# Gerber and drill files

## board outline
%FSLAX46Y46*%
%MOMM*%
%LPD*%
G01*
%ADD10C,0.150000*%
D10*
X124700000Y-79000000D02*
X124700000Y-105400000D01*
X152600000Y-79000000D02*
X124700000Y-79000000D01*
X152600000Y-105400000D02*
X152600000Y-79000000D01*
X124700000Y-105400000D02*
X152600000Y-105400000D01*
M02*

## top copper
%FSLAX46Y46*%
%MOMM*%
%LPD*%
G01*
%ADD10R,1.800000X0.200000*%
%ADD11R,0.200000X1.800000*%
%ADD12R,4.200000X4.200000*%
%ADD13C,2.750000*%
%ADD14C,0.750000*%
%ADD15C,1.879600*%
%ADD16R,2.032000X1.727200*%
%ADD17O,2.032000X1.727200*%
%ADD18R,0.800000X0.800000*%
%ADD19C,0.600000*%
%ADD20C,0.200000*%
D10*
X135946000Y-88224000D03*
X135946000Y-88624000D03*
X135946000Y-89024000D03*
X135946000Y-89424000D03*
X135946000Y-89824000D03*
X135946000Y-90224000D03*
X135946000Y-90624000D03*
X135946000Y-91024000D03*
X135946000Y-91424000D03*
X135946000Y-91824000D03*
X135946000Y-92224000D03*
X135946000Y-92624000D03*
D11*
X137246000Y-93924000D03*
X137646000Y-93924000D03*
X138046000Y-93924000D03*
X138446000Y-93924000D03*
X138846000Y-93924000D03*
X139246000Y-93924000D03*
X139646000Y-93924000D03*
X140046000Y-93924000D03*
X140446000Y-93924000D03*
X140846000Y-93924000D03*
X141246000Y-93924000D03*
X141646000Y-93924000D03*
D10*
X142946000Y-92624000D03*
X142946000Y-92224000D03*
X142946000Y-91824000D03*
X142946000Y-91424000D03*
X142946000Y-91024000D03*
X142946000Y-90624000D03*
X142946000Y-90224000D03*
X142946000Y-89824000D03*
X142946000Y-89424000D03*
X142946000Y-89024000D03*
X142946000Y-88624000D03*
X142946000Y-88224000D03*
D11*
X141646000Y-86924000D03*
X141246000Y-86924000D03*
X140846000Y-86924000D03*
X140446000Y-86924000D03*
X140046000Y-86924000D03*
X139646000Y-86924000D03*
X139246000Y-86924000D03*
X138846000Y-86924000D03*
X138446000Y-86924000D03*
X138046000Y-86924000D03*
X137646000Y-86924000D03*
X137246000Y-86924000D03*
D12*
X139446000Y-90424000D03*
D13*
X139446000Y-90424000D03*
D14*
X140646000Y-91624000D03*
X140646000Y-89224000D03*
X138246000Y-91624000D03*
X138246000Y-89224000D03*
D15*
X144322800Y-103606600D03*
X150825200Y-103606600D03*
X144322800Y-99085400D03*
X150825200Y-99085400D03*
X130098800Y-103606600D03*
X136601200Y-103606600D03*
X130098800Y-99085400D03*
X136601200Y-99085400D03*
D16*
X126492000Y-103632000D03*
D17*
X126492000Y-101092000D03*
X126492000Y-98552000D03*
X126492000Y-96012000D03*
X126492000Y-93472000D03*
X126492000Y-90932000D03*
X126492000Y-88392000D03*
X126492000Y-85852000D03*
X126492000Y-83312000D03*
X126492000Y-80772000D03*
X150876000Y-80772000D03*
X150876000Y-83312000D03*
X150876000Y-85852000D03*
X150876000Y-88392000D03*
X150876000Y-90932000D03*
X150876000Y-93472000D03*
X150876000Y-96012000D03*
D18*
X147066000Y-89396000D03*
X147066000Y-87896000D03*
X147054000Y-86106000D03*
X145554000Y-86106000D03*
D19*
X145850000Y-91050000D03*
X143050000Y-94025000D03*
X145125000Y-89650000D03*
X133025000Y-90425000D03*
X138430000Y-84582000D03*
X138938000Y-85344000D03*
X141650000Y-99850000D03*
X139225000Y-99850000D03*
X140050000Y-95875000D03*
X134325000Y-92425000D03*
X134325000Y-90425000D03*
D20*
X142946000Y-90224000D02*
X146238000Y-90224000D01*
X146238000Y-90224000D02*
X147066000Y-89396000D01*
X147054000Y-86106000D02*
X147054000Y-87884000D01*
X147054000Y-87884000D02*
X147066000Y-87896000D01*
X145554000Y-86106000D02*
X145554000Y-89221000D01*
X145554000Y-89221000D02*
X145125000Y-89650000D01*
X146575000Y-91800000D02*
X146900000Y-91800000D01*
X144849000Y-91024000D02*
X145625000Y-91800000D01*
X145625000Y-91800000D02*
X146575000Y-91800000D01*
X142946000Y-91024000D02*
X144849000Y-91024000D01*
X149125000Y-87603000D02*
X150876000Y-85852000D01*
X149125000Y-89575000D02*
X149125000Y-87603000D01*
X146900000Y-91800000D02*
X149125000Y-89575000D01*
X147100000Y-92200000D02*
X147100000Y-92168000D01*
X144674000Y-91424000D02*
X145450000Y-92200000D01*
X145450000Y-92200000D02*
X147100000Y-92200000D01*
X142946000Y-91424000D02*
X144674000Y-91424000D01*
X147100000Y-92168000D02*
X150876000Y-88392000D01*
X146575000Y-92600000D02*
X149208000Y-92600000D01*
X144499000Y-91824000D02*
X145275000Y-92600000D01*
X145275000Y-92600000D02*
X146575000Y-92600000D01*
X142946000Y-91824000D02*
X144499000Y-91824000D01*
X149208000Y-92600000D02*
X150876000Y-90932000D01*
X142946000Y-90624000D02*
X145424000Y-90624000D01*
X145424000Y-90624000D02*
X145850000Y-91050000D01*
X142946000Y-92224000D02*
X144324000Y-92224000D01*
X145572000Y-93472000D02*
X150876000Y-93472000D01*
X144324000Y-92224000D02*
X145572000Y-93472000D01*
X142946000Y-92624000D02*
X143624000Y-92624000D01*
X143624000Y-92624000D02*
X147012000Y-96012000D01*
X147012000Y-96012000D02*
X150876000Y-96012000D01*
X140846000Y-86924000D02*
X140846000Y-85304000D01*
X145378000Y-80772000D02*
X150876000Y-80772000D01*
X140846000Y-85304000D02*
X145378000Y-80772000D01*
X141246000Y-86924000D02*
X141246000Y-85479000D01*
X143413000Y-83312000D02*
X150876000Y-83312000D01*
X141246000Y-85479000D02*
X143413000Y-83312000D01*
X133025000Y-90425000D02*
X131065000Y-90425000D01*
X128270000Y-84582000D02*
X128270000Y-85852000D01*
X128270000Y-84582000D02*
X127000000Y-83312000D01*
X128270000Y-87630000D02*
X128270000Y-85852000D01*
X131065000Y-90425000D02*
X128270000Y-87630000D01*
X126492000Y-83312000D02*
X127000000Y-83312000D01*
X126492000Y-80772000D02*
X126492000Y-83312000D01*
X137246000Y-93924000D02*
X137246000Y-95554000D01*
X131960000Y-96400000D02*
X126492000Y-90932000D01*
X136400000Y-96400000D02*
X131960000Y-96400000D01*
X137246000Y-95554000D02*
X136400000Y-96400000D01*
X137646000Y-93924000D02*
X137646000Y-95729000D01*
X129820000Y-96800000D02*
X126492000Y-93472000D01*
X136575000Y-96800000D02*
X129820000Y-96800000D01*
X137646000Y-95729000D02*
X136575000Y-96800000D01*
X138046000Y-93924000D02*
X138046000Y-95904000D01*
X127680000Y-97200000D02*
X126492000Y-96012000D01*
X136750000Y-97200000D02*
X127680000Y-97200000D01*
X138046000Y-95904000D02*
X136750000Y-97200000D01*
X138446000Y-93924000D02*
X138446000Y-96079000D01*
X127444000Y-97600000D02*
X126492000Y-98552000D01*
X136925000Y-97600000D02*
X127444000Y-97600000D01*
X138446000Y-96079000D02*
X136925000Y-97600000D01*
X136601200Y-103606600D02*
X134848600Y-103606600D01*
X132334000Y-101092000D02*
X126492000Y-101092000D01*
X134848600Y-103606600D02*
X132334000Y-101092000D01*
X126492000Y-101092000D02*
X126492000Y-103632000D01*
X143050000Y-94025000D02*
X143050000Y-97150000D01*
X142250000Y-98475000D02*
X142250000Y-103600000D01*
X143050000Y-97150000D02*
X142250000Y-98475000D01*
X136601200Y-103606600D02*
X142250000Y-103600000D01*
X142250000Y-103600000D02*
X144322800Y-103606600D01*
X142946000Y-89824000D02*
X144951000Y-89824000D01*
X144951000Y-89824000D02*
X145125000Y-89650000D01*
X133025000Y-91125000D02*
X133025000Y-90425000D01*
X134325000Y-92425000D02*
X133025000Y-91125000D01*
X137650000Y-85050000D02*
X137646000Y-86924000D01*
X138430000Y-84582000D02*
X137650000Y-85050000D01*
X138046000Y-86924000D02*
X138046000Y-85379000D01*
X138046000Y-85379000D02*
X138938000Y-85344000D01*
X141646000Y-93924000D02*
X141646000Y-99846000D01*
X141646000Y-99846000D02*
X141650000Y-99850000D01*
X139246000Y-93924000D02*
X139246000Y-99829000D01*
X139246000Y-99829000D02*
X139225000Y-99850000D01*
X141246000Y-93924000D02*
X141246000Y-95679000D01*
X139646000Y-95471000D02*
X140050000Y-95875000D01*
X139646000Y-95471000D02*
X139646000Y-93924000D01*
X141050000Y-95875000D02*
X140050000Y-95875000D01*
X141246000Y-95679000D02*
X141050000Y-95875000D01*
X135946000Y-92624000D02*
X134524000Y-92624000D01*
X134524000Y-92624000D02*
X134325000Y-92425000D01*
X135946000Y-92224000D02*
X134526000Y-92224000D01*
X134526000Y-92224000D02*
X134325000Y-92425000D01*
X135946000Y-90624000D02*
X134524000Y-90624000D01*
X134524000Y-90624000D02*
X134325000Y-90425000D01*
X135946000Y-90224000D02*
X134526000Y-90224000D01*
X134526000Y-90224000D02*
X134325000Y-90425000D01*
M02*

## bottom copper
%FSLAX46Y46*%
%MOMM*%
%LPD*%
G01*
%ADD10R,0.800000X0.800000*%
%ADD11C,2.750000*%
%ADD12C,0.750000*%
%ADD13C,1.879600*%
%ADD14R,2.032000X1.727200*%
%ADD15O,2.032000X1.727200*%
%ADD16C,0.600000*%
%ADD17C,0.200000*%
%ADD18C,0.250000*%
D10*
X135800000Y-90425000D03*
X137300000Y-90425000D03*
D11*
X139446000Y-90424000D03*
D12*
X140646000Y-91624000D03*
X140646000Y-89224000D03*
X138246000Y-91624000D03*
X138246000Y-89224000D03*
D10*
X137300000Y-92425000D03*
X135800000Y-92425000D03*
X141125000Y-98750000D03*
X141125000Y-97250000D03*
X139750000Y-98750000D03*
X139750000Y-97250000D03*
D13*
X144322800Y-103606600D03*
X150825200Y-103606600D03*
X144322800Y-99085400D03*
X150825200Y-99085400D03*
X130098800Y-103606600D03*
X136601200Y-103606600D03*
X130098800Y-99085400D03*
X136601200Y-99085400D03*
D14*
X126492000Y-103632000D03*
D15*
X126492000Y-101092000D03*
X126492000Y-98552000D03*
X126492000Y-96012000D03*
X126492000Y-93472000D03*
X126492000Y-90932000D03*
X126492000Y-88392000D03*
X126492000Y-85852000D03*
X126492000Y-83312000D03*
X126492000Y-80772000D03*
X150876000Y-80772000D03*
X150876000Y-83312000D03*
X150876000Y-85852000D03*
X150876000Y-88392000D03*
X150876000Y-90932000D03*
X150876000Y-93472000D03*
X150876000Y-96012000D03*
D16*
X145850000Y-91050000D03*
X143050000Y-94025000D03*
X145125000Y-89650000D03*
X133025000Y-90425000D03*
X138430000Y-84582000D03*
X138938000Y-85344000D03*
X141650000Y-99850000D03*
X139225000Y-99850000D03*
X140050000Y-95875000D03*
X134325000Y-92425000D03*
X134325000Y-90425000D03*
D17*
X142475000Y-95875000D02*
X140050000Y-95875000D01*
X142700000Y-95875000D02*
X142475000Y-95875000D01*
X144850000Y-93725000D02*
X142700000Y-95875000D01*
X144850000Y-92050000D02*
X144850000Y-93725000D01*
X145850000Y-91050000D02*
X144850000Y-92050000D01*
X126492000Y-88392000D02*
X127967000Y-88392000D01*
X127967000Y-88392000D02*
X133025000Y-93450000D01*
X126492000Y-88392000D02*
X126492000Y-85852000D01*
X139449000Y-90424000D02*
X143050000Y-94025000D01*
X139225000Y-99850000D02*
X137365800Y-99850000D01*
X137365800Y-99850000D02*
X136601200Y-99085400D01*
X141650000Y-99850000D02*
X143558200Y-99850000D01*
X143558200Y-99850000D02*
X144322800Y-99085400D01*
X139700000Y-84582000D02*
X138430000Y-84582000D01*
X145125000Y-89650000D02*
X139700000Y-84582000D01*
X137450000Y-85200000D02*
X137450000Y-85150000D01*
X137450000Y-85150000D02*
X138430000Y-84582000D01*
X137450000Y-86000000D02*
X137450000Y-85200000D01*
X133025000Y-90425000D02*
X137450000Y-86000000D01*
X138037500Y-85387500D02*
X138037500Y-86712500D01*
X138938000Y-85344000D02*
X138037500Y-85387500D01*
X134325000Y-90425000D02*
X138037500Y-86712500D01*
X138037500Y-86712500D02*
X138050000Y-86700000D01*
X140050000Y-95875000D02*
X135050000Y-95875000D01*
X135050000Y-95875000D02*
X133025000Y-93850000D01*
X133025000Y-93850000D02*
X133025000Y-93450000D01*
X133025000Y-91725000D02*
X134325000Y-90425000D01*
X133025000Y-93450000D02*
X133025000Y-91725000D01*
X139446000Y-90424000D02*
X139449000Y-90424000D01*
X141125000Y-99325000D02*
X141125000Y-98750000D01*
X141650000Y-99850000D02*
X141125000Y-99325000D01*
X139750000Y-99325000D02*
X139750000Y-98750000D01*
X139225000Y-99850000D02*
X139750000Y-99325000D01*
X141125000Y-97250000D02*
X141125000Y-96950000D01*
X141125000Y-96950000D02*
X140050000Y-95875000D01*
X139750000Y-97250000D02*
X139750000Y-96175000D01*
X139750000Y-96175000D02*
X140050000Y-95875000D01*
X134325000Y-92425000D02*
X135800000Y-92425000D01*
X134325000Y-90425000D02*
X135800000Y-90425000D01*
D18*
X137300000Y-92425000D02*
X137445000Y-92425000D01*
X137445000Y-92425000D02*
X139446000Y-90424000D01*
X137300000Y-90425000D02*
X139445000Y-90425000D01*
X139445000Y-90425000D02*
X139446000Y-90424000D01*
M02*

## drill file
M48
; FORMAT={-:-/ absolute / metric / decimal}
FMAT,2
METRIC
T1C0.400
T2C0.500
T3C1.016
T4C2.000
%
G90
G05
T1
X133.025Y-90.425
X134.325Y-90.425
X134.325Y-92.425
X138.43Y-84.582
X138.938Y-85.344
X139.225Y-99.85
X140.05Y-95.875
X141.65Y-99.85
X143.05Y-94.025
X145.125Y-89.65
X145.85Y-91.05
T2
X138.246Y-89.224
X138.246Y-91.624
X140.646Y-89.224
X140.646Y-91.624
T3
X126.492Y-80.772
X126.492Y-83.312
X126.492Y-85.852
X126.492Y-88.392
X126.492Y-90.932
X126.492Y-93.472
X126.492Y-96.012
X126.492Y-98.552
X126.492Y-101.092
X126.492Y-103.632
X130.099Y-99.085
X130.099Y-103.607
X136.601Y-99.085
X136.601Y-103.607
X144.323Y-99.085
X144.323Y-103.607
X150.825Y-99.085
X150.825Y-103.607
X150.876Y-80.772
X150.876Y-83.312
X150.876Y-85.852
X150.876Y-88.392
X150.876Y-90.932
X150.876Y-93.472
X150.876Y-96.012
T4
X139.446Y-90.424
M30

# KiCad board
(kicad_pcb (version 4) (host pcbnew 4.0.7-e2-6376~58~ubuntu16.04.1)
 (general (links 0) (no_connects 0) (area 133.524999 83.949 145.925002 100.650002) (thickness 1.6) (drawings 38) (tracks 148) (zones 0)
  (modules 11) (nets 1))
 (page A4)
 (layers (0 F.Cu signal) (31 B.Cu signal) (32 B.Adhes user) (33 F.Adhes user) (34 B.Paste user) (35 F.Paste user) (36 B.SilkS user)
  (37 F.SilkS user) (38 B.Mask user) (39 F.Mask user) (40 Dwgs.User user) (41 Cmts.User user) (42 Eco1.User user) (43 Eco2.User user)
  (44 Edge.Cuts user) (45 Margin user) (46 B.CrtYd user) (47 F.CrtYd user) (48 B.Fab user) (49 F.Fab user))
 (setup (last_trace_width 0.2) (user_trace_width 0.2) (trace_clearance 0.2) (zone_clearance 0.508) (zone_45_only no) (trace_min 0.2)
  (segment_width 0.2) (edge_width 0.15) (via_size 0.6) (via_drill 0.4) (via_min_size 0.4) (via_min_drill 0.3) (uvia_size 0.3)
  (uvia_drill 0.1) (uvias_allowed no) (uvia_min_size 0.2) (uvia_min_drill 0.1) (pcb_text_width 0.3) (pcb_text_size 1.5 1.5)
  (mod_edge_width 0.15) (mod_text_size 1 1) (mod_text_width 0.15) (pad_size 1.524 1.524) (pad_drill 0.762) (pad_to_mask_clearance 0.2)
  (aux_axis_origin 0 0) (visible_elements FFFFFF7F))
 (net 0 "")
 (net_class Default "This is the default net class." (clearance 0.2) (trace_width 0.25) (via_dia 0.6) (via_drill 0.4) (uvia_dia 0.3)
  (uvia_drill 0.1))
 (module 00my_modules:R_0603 (layer B.Cu) (at 136.55 90.425)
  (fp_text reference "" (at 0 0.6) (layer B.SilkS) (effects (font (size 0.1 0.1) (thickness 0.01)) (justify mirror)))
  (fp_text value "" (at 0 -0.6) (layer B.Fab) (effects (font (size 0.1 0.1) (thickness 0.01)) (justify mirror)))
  (pad 1 smd rect (at -0.75 0) (size 0.8 0.8) (layers B.Cu B.Paste B.Mask))
  (pad 2 smd rect (at 0.75 0) (size 0.8 0.8) (layers B.Cu B.Paste B.Mask)))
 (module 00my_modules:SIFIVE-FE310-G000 (layer F.Cu) (at 139.446 90.424)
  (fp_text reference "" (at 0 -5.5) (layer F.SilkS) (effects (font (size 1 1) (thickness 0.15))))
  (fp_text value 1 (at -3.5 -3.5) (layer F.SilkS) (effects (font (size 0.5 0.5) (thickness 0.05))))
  (pad DQ3 smd rect (at -3.5 -2.2) (size 1.8 0.2) (layers F.Cu F.Paste F.Mask))
  (pad DQ2 smd rect (at -3.5 -1.8) (size 1.8 0.2) (layers F.Cu F.Paste F.Mask))
  (pad DQ1 smd rect (at -3.5 -1.4) (size 1.8 0.2) (layers F.Cu F.Paste F.Mask))
  (pad DQ0 smd rect (at -3.5 -1) (size 1.8 0.2) (layers F.Cu F.Paste F.Mask))
  (pad CS smd rect (at -3.5 -0.6) (size 1.8 0.2) (layers F.Cu F.Paste F.Mask))
  (pad 1.8V smd rect (at -3.5 -0.2) (size 1.8 0.2) (layers F.Cu F.Paste F.Mask))
  (pad 1.8V smd rect (at -3.5 0.2) (size 1.8 0.2) (layers F.Cu F.Paste F.Mask))
  (pad PLL smd rect (at -3.5 0.6) (size 1.8 0.2) (layers F.Cu F.Paste F.Mask))
  (pad XIN smd rect (at -3.5 1) (size 1.8 0.2) (layers F.Cu F.Paste F.Mask))
  (pad NC smd rect (at -3.5 1.4) (size 1.8 0.2) (layers F.Cu F.Paste F.Mask))
  (pad 3.3V smd rect (at -3.5 1.8) (size 1.8 0.2) (layers F.Cu F.Paste F.Mask))
  (pad 3.3V smd rect (at -3.5 2.2) (size 1.8 0.2) (layers F.Cu F.Paste F.Mask))
  (pad TCK smd rect (at -2.2 3.5 90) (size 1.8 0.2) (layers F.Cu F.Paste F.Mask))
  (pad TDO smd rect (at -1.8 3.5 90) (size 1.8 0.2) (layers F.Cu F.Paste F.Mask))
  (pad TMS smd rect (at -1.4 3.5 90) (size 1.8 0.2) (layers F.Cu F.Paste F.Mask))
  (pad TDI smd rect (at -1 3.5 90) (size 1.8 0.2) (layers F.Cu F.Paste F.Mask))
  (pad 17 smd rect (at -0.6 3.5 90) (size 1.8 0.2) (layers F.Cu F.Paste F.Mask))
  (pad WAKE smd rect (at -0.2 3.5 90) (size 1.8 0.2) (layers F.Cu F.Paste F.Mask))
  (pad 1.8V smd rect (at 0.2 3.5 90) (size 1.8 0.2) (layers F.Cu F.Paste F.Mask))
  (pad 20 smd rect (at 0.6 3.5 90) (size 1.8 0.2) (layers F.Cu F.Paste F.Mask))
  (pad 21 smd rect (at 1 3.5 90) (size 1.8 0.2) (layers F.Cu F.Paste F.Mask))
  (pad 22 smd rect (at 1.4 3.5 90) (size 1.8 0.2) (layers F.Cu F.Paste F.Mask))
  (pad 1.8V smd rect (at 1.8 3.5 90) (size 1.8 0.2) (layers F.Cu F.Paste F.Mask))
  (pad ERST smd rect (at 2.2 3.5 90) (size 1.8 0.2) (layers F.Cu F.Paste F.Mask))
  (pad G00 smd rect (at 3.5 2.2) (size 1.8 0.2) (layers F.Cu F.Paste F.Mask))
  (pad G01 smd rect (at 3.5 1.8) (size 1.8 0.2) (layers F.Cu F.Paste F.Mask))
  (pad G02 smd rect (at 3.5 1.4) (size 1.8 0.2) (layers F.Cu F.Paste F.Mask))
  (pad G03 smd rect (at 3.5 1) (size 1.8 0.2) (layers F.Cu F.Paste F.Mask))
  (pad G04 smd rect (at 3.5 0.6) (size 1.8 0.2) (layers F.Cu F.Paste F.Mask))
  (pad 1.8V smd rect (at 3.5 0.2) (size 1.8 0.2) (layers F.Cu F.Paste F.Mask))
  (pad G05 smd rect (at 3.5 -0.2) (size 1.8 0.2) (layers F.Cu F.Paste F.Mask))
  (pad 3.3V smd rect (at 3.5 -0.6) (size 1.8 0.2) (layers F.Cu F.Paste F.Mask))
  (pad G09 smd rect (at 3.5 -1) (size 1.8 0.2) (layers F.Cu F.Paste F.Mask))
  (pad G10 smd rect (at 3.5 -1.4) (size 1.8 0.2) (layers F.Cu F.Paste F.Mask))
  (pad G11 smd rect (at 3.5 -1.8) (size 1.8 0.2) (layers F.Cu F.Paste F.Mask))
  (pad G12 smd rect (at 3.5 -2.2) (size 1.8 0.2) (layers F.Cu F.Paste F.Mask))
  (pad G13 smd rect (at 2.2 -3.5 90) (size 1.8 0.2) (layers F.Cu F.Paste F.Mask))
  (pad RX smd rect (at 1.8 -3.5 90) (size 1.8 0.2) (layers F.Cu F.Paste F.Mask))
  (pad TX smd rect (at 1.4 -3.5 90) (size 1.8 0.2) (layers F.Cu F.Paste F.Mask))
  (pad G18 smd rect (at 1 -3.5 90) (size 1.8 0.2) (layers F.Cu F.Paste F.Mask))
  (pad G19 smd rect (at 0.6 -3.5 90) (size 1.8 0.2) (layers F.Cu F.Paste F.Mask))
  (pad G20 smd rect (at 0.2 -3.5 90) (size 1.8 0.2) (layers F.Cu F.Paste F.Mask))
  (pad G21 smd rect (at -0.2 -3.5 90) (size 1.8 0.2) (layers F.Cu F.Paste F.Mask))
  (pad G22 smd rect (at -0.6 -3.5 90) (size 1.8 0.2) (layers F.Cu F.Paste F.Mask))
  (pad G23 smd rect (at -1 -3.5 90) (size 1.8 0.2) (layers F.Cu F.Paste F.Mask))
  (pad 1.8V smd rect (at -1.4 -3.5 90) (size 1.8 0.2) (layers F.Cu F.Paste F.Mask))
  (pad 3.3V smd rect (at -1.8 -3.5 90) (size 1.8 0.2) (layers F.Cu F.Paste F.Mask))
  (pad SCK smd rect (at -2.2 -3.5 90) (size 1.8 0.2) (layers F.Cu F.Paste F.Mask))
  (pad GND smd rect (at 0 0) (size 4.2 4.2) (layers F.Cu F.Paste F.Mask))
  (pad "" thru_hole circle (at 0 0) (size 2.75 2.75) (drill 2) (layers *.Cu *.Mask F.SilkS))
  (pad "" thru_hole circle (at 1.2 1.2) (size 0.75 0.75) (drill 0.5) (layers *.Cu *.Mask F.SilkS))
  (pad "" thru_hole circle (at 1.2 -1.2) (size 0.75 0.75) (drill 0.5) (layers *.Cu *.Mask F.SilkS))
  (pad "" thru_hole circle (at -1.2 1.2) (size 0.75 0.75) (drill 0.5) (layers *.Cu *.Mask F.SilkS))
  (pad "" thru_hole circle (at -1.2 -1.2) (size 0.75 0.75) (drill 0.5) (layers *.Cu *.Mask F.SilkS)))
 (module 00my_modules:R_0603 (layer B.Cu) (at 136.55 92.425 180)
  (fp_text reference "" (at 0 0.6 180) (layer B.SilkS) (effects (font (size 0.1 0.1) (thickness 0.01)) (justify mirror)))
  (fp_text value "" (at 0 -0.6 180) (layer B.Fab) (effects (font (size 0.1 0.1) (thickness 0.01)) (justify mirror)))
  (pad 1 smd rect (at -0.75 0 180) (size 0.8 0.8) (layers B.Cu B.Paste B.Mask))
  (pad 2 smd rect (at 0.75 0 180) (size 0.8 0.8) (layers B.Cu B.Paste B.Mask)))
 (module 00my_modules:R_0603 (layer B.Cu) (at 141.125 98 90)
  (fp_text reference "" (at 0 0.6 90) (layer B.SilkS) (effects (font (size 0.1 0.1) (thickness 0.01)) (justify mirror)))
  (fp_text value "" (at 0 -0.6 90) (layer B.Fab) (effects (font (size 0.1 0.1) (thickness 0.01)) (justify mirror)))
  (pad 1 smd rect (at -0.75 0 90) (size 0.8 0.8) (layers B.Cu B.Paste B.Mask))
  (pad 2 smd rect (at 0.75 0 90) (size 0.8 0.8) (layers B.Cu B.Paste B.Mask)))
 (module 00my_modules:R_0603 (layer B.Cu) (at 139.75 98 90)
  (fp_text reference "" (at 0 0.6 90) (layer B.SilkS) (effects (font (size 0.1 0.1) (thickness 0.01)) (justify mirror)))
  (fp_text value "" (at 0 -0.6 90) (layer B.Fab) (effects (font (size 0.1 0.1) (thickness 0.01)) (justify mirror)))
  (pad 1 smd rect (at -0.75 0 90) (size 0.8 0.8) (layers B.Cu B.Paste B.Mask))
  (pad 2 smd rect (at 0.75 0 90) (size 0.8 0.8) (layers B.Cu B.Paste B.Mask)))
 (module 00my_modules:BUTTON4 (layer F.Cu) (at 147.574 101.346)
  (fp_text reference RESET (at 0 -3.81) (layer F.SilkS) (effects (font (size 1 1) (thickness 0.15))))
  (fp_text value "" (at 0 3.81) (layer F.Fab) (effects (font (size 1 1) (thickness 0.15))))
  (pad 1 thru_hole circle (at -3.2512 2.2606) (size 1.8796 1.8796) (drill 1.016) (layers *.Cu *.Mask F.SilkS))
  (pad 2 thru_hole circle (at 3.2512 2.2606) (size 1.8796 1.8796) (drill 1.016) (layers *.Cu *.Mask F.SilkS))
  (pad 3 thru_hole circle (at -3.2512 -2.2606) (size 1.8796 1.8796) (drill 1.016) (layers *.Cu *.Mask F.SilkS))
  (pad 4 thru_hole circle (at 3.2512 -2.2606) (size 1.8796 1.8796) (drill 1.016) (layers *.Cu *.Mask F.SilkS)))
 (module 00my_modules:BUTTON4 (layer F.Cu) (at 133.35 101.346)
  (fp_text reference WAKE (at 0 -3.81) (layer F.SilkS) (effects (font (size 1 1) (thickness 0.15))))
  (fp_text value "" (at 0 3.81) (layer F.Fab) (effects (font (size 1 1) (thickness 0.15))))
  (pad 1 thru_hole circle (at -3.2512 2.2606) (size 1.8796 1.8796) (drill 1.016) (layers *.Cu *.Mask F.SilkS))
  (pad 2 thru_hole circle (at 3.2512 2.2606) (size 1.8796 1.8796) (drill 1.016) (layers *.Cu *.Mask F.SilkS))
  (pad 3 thru_hole circle (at -3.2512 -2.2606) (size 1.8796 1.8796) (drill 1.016) (layers *.Cu *.Mask F.SilkS))
  (pad 4 thru_hole circle (at 3.2512 -2.2606) (size 1.8796 1.8796) (drill 1.016) (layers *.Cu *.Mask F.SilkS)))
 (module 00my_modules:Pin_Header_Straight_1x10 (layer F.Cu) (at 126.492 103.632 180)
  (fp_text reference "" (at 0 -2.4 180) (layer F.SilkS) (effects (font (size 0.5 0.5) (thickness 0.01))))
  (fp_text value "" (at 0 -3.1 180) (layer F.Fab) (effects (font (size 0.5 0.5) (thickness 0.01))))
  (pad 1 thru_hole rect (at 0 0 180) (size 2.032 1.7272) (drill 1.016) (layers *.Cu *.Mask F.SilkS))
  (pad 2 thru_hole oval (at 0 2.54 180) (size 2.032 1.7272) (drill 1.016) (layers *.Cu *.Mask F.SilkS))
  (pad 3 thru_hole oval (at 0 5.08 180) (size 2.032 1.7272) (drill 1.016) (layers *.Cu *.Mask F.SilkS))
  (pad 4 thru_hole oval (at 0 7.62 180) (size 2.032 1.7272) (drill 1.016) (layers *.Cu *.Mask F.SilkS))
  (pad 5 thru_hole oval (at 0 10.16 180) (size 2.032 1.7272) (drill 1.016) (layers *.Cu *.Mask F.SilkS))
  (pad 6 thru_hole oval (at 0 12.7 180) (size 2.032 1.7272) (drill 1.016) (layers *.Cu *.Mask F.SilkS))
  (pad 7 thru_hole oval (at 0 15.24 180) (size 2.032 1.7272) (drill 1.016) (layers *.Cu *.Mask F.SilkS))
  (pad 8 thru_hole oval (at 0 17.78 180) (size 2.032 1.7272) (drill 1.016) (layers *.Cu *.Mask F.SilkS))
  (pad 9 thru_hole oval (at 0 20.32 180) (size 2.032 1.7272) (drill 1.016) (layers *.Cu *.Mask F.SilkS))
  (pad 10 thru_hole oval (at 0 22.86 180) (size 2.032 1.7272) (drill 1.016) (layers *.Cu *.Mask F.SilkS)))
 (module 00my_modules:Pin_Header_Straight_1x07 (layer F.Cu) (at 150.876 80.772)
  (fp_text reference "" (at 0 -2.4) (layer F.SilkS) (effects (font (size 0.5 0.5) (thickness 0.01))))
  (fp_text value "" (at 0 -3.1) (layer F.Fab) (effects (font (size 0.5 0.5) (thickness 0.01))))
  (pad 1 thru_hole oval (at 0 0) (size 2.032 1.7272) (drill 1.016) (layers *.Cu *.Mask F.SilkS))
  (pad 2 thru_hole oval (at 0 2.54) (size 2.032 1.7272) (drill 1.016) (layers *.Cu *.Mask F.SilkS))
  (pad 3 thru_hole oval (at 0 5.08) (size 2.032 1.7272) (drill 1.016) (layers *.Cu *.Mask F.SilkS))
  (pad 4 thru_hole oval (at 0 7.62) (size 2.032 1.7272) (drill 1.016) (layers *.Cu *.Mask F.SilkS))
  (pad 5 thru_hole oval (at 0 10.16) (size 2.032 1.7272) (drill 1.016) (layers *.Cu *.Mask F.SilkS))
  (pad 6 thru_hole oval (at 0 12.7) (size 2.032 1.7272) (drill 1.016) (layers *.Cu *.Mask F.SilkS))
  (pad 7 thru_hole oval (at 0 15.24) (size 2.032 1.7272) (drill 1.016) (layers *.Cu *.Mask F.SilkS)))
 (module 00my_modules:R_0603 (layer F.Cu) (at 147.066 88.646 90)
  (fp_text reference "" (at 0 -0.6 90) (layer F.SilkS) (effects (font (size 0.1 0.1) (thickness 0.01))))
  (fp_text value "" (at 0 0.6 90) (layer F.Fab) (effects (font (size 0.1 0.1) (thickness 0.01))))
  (pad 1 smd rect (at -0.75 0 90) (size 0.8 0.8) (layers F.Cu F.Paste F.Mask))
  (pad 2 smd rect (at 0.75 0 90) (size 0.8 0.8) (layers F.Cu F.Paste F.Mask)))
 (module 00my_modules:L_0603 (layer F.Cu) (at 146.304 86.106 180)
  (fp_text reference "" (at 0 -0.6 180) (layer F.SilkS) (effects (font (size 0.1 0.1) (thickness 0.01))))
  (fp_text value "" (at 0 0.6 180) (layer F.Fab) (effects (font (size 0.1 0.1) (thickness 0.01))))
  (pad 1 smd rect (at -0.75 0 180) (size 0.8 0.8) (layers F.Cu F.Paste F.Mask))
  (pad 2 smd rect (at 0.75 0 180) (size 0.8 0.8) (layers F.Cu F.Paste F.Mask)))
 (gr_line (start 124.7 79) (end 124.7 105.4) (angle 90) (layer Edge.Cuts) (width 0.15))
 (gr_line (start 152.6 79) (end 124.7 79) (angle 90) (layer Edge.Cuts) (width 0.15))
 (gr_line (start 152.6 105.4) (end 152.6 79) (angle 90) (layer Edge.Cuts) (width 0.15))
 (gr_line (start 124.7 105.4) (end 152.6 105.4) (angle 90) (layer Edge.Cuts) (width 0.15))
 (segment (start 142.946 90.224) (end 146.238 90.224) (width 0.2) (layer F.Cu) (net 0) (status 400000))
 (segment (start 146.238 90.224) (end 147.066 89.396) (width 0.2) (layer F.Cu) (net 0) (status 800000))
 (segment (start 147.054 86.106) (end 147.054 87.884) (width 0.2) (layer F.Cu) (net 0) (status C00000))
 (segment (start 147.054 87.884) (end 147.066 87.896) (width 0.2) (layer F.Cu) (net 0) (status C00000))
 (segment (start 145.554 86.106) (end 145.554 89.221) (width 0.2) (layer F.Cu) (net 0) (status 400000))
 (segment (start 145.554 89.221) (end 145.125 89.65) (width 0.2) (layer F.Cu) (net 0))
 (segment (start 146.575 91.8) (end 146.9 91.8) (width 0.2) (layer F.Cu) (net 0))
 (segment (start 144.849 91.024) (end 145.625 91.8) (width 0.2) (layer F.Cu) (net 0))
 (segment (start 145.625 91.8) (end 146.575 91.8) (width 0.2) (layer F.Cu) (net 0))
 (segment (start 142.946 91.024) (end 144.849 91.024) (width 0.2) (layer F.Cu) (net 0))
 (segment (start 149.125 87.603) (end 150.876 85.852) (width 0.2) (layer F.Cu) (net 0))
 (segment (start 149.125 89.575) (end 149.125 87.603) (width 0.2) (layer F.Cu) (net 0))
 (segment (start 146.9 91.8) (end 149.125 89.575) (width 0.2) (layer F.Cu) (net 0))
 (segment (start 147.1 92.2) (end 147.1 92.168) (width 0.2) (layer F.Cu) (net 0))
 (segment (start 144.674 91.424) (end 145.45 92.2) (width 0.2) (layer F.Cu) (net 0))
 (segment (start 145.45 92.2) (end 147.1 92.2) (width 0.2) (layer F.Cu) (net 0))
 (segment (start 142.946 91.424) (end 144.674 91.424) (width 0.2) (layer F.Cu) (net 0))
 (segment (start 147.1 92.168) (end 150.876 88.392) (width 0.2) (layer F.Cu) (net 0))
 (segment (start 146.575 92.6) (end 149.208 92.6) (width 0.2) (layer F.Cu) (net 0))
 (segment (start 144.499 91.824) (end 145.275 92.6) (width 0.2) (layer F.Cu) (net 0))
 (segment (start 145.275 92.6) (end 146.575 92.6) (width 0.2) (layer F.Cu) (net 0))
 (segment (start 142.946 91.824) (end 144.499 91.824) (width 0.2) (layer F.Cu) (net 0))
 (segment (start 149.208 92.6) (end 150.876 90.932) (width 0.2) (layer F.Cu) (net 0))
 (segment (start 142.946 90.624) (end 145.424 90.624) (width 0.2) (layer F.Cu) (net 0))
 (segment (start 142.475 95.875) (end 140.05 95.875) (width 0.2) (layer B.Cu) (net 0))
 (segment (start 142.7 95.875) (end 142.475 95.875) (width 0.2) (layer B.Cu) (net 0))
 (segment (start 144.85 93.725) (end 142.7 95.875) (width 0.2) (layer B.Cu) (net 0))
 (segment (start 144.85 92.05) (end 144.85 93.725) (width 0.2) (layer B.Cu) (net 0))
 (segment (start 145.85 91.05) (end 144.85 92.05) (width 0.2) (layer B.Cu) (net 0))
 (via (at 145.85 91.05) (size 0.6) (drill 0.4) (layers F.Cu B.Cu) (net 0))
 (segment (start 145.424 90.624) (end 145.85 91.05) (width 0.2) (layer F.Cu) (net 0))
 (segment (start 142.946 92.224) (end 144.324 92.224) (width 0.2) (layer F.Cu) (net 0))
 (segment (start 145.572 93.472) (end 150.876 93.472) (width 0.2) (layer F.Cu) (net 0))
 (segment (start 144.324 92.224) (end 145.572 93.472) (width 0.2) (layer F.Cu) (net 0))
 (segment (start 142.946 92.624) (end 143.624 92.624) (width 0.2) (layer F.Cu) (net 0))
 (segment (start 143.624 92.624) (end 147.012 96.012) (width 0.2) (layer F.Cu) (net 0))
 (segment (start 147.012 96.012) (end 150.876 96.012) (width 0.2) (layer F.Cu) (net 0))
 (segment (start 140.846 86.924) (end 140.846 85.304) (width 0.2) (layer F.Cu) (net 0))
 (segment (start 145.378 80.772) (end 150.876 80.772) (width 0.2) (layer F.Cu) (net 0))
 (segment (start 140.846 85.304) (end 145.378 80.772) (width 0.2) (layer F.Cu) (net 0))
 (segment (start 141.246 86.924) (end 141.246 85.479) (width 0.2) (layer F.Cu) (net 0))
 (segment (start 143.413 83.312) (end 150.876 83.312) (width 0.2) (layer F.Cu) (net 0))
 (segment (start 141.246 85.479) (end 143.413 83.312) (width 0.2) (layer F.Cu) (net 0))
 (segment (start 133.025 90.425) (end 131.065 90.425) (width 0.2) (layer F.Cu) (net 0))
 (segment (start 128.27 84.582) (end 128.27 85.852) (width 0.2) (layer F.Cu) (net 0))
 (segment (start 128.27 84.582) (end 127 83.312) (width 0.2) (layer F.Cu) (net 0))
 (segment (start 128.27 87.63) (end 128.27 85.852) (width 0.2) (layer F.Cu) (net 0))
 (segment (start 131.065 90.425) (end 128.27 87.63) (width 0.2) (layer F.Cu) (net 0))
 (segment (start 126.492 83.312) (end 127 83.312) (width 0.2) (layer F.Cu) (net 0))
 (segment (start 126.492 80.772) (end 126.492 83.312) (width 0.2) (layer F.Cu) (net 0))
 (segment (start 126.492 88.392) (end 127.967 88.392) (width 0.2) (layer B.Cu) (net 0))
 (segment (start 127.967 88.392) (end 133.025 93.45) (width 0.2) (layer B.Cu) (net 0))
 (segment (start 126.492 88.392) (end 126.492 85.852) (width 0.2) (layer B.Cu) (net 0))
 (segment (start 137.246 93.924) (end 137.246 95.554) (width 0.2) (layer F.Cu) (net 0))
 (segment (start 131.96 96.4) (end 126.492 90.932) (width 0.2) (layer F.Cu) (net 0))
 (segment (start 136.4 96.4) (end 131.96 96.4) (width 0.2) (layer F.Cu) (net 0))
 (segment (start 137.246 95.554) (end 136.4 96.4) (width 0.2) (layer F.Cu) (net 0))
 (segment (start 137.646 93.924) (end 137.646 95.729) (width 0.2) (layer F.Cu) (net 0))
 (segment (start 129.82 96.8) (end 126.492 93.472) (width 0.2) (layer F.Cu) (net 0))
 (segment (start 136.575 96.8) (end 129.82 96.8) (width 0.2) (layer F.Cu) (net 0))
 (segment (start 137.646 95.729) (end 136.575 96.8) (width 0.2) (layer F.Cu) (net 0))
 (segment (start 138.046 93.924) (end 138.046 95.904) (width 0.2) (layer F.Cu) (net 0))
 (segment (start 127.68 97.2) (end 126.492 96.012) (width 0.2) (layer F.Cu) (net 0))
 (segment (start 136.75 97.2) (end 127.68 97.2) (width 0.2) (layer F.Cu) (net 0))
 (segment (start 138.046 95.904) (end 136.75 97.2) (width 0.2) (layer F.Cu) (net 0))
 (segment (start 138.446 93.924) (end 138.446 96.079) (width 0.2) (layer F.Cu) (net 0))
 (segment (start 127.444 97.6) (end 126.492 98.552) (width 0.2) (layer F.Cu) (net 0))
 (segment (start 136.925 97.6) (end 127.444 97.6) (width 0.2) (layer F.Cu) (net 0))
 (segment (start 138.446 96.079) (end 136.925 97.6) (width 0.2) (layer F.Cu) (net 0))
 (segment (start 136.6012 103.6066) (end 134.8486 103.6066) (width 0.2) (layer F.Cu) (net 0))
 (segment (start 132.334 101.092) (end 126.492 101.092) (width 0.2) (layer F.Cu) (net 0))
 (segment (start 134.8486 103.6066) (end 132.334 101.092) (width 0.2) (layer F.Cu) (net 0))
 (segment (start 126.492 101.092) (end 126.492 103.632) (width 0.2) (layer F.Cu) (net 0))
 (segment (start 143.05 94.025) (end 143.05 97.15) (width 0.2) (layer F.Cu) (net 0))
 (via (at 143.05 94.025) (size 0.6) (drill 0.4) (layers F.Cu B.Cu) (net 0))
 (segment (start 139.449 90.424) (end 143.05 94.025) (width 0.2) (layer B.Cu) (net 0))
 (segment (start 142.25 98.475) (end 142.25 103.6) (width 0.2) (layer F.Cu) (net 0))
 (segment (start 143.05 97.15) (end 142.25 98.475) (width 0.2) (layer F.Cu) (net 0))
 (segment (start 136.6012 103.6066) (end 142.25 103.6) (width 0.2) (layer F.Cu) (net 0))
 (segment (start 142.25 103.6) (end 144.3228 103.6066) (width 0.2) (layer F.Cu) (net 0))
 (segment (start 139.225 99.85) (end 137.3658 99.85) (width 0.2) (layer B.Cu) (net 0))
 (segment (start 137.3658 99.85) (end 136.6012 99.0854) (width 0.2) (layer B.Cu) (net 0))
 (segment (start 141.65 99.85) (end 143.5582 99.85) (width 0.2) (layer B.Cu) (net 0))
 (segment (start 143.5582 99.85) (end 144.3228 99.0854) (width 0.2) (layer B.Cu) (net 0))
 (segment (start 142.946 89.824) (end 144.951 89.824) (width 0.2) (layer F.Cu) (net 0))
 (segment (start 139.7 84.582) (end 138.43 84.582) (width 0.2) (layer B.Cu) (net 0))
 (segment (start 145.125 89.65) (end 139.7 84.582) (width 0.2) (layer B.Cu) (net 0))
 (via (at 145.125 89.65) (size 0.6) (drill 0.4) (layers F.Cu B.Cu) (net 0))
 (segment (start 144.951 89.824) (end 145.125 89.65) (width 0.2) (layer F.Cu) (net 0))
 (segment (start 137.45 85.2) (end 137.45 85.15) (width 0.2) (layer B.Cu) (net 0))
 (segment (start 137.45 85.15) (end 138.43 84.582) (width 0.2) (layer B.Cu) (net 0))
 (segment (start 137.45 86) (end 137.45 85.2) (width 0.2) (layer B.Cu) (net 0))
 (segment (start 133.025 90.425) (end 137.45 86) (width 0.2) (layer B.Cu) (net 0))
 (via (at 133.025 90.425) (size 0.6) (drill 0.4) (layers F.Cu B.Cu) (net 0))
 (segment (start 133.025 91.125) (end 133.025 90.425) (width 0.2) (layer F.Cu) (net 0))
 (segment (start 134.325 92.425) (end 133.025 91.125) (width 0.2) (layer F.Cu) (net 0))
 (segment (start 137.65 85.05) (end 137.646 86.924) (width 0.2) (layer F.Cu) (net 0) (status 800000))
 (segment (start 138.43 84.582) (end 137.65 85.05) (width 0.2) (layer F.Cu) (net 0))
 (via (at 138.43 84.582) (size 0.6) (drill 0.4) (layers F.Cu B.Cu) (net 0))
 (segment (start 138.046 86.924) (end 138.046 85.379) (width 0.2) (layer F.Cu) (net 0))
 (segment (start 138.0375 85.3875) (end 138.0375 86.7125) (width 0.2) (layer B.Cu) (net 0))
 (segment (start 138.938 85.344) (end 138.0375 85.3875) (width 0.2) (layer B.Cu) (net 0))
 (via (at 138.938 85.344) (size 0.6) (drill 0.4) (layers F.Cu B.Cu) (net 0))
 (segment (start 138.046 85.379) (end 138.938 85.344) (width 0.2) (layer F.Cu) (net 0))
 (segment (start 134.325 90.425) (end 138.0375 86.7125) (width 0.2) (layer B.Cu) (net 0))
 (segment (start 138.0375 86.7125) (end 138.05 86.7) (width 0.2) (layer B.Cu) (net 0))
 (segment (start 140.05 95.875) (end 135.05 95.875) (width 0.2) (layer B.Cu) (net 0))
 (segment (start 135.05 95.875) (end 133.025 93.85) (width 0.2) (layer B.Cu) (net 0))
 (segment (start 133.025 93.85) (end 133.025 93.45) (width 0.2) (layer B.Cu) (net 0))
 (segment (start 133.025 91.725) (end 134.325 90.425) (width 0.2) (layer B.Cu) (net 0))
 (segment (start 133.025 93.45) (end 133.025 91.725) (width 0.2) (layer B.Cu) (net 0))
 (segment (start 139.446 90.424) (end 139.449 90.424) (width 0.2) (layer B.Cu) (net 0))
 (segment (start 141.646 93.924) (end 141.646 99.846) (width 0.2) (layer F.Cu) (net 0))
 (segment (start 141.125 99.325) (end 141.125 98.75) (width 0.2) (layer B.Cu) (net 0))
 (segment (start 141.65 99.85) (end 141.125 99.325) (width 0.2) (layer B.Cu) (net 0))
 (via (at 141.65 99.85) (size 0.6) (drill 0.4) (layers F.Cu B.Cu) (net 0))
 (segment (start 141.646 99.846) (end 141.65 99.85) (width 0.2) (layer F.Cu) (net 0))
 (segment (start 139.246 93.924) (end 139.246 99.829) (width 0.2) (layer F.Cu) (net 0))
 (segment (start 139.75 99.325) (end 139.75 98.75) (width 0.2) (layer B.Cu) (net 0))
 (segment (start 139.225 99.85) (end 139.75 99.325) (width 0.2) (layer B.Cu) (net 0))
 (via (at 139.225 99.85) (size 0.6) (drill 0.4) (layers F.Cu B.Cu) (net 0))
 (segment (start 139.246 99.829) (end 139.225 99.85) (width 0.2) (layer F.Cu) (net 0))
 (segment (start 141.125 97.25) (end 141.125 96.95) (width 0.2) (layer B.Cu) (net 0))
 (segment (start 141.125 96.95) (end 140.05 95.875) (width 0.2) (layer B.Cu) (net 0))
 (segment (start 139.75 97.25) (end 139.75 96.175) (width 0.2) (layer B.Cu) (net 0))
 (via (at 140.05 95.875) (size 0.6) (drill 0.4) (layers F.Cu B.Cu) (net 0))
 (segment (start 139.75 96.175) (end 140.05 95.875) (width 0.2) (layer B.Cu) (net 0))
 (segment (start 141.246 93.924) (end 141.246 95.679) (width 0.2) (layer F.Cu) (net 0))
 (segment (start 139.646 95.471) (end 140.05 95.875) (width 0.2) (layer F.Cu) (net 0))
 (segment (start 139.646 95.471) (end 139.646 93.924) (width 0.2) (layer F.Cu) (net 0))
 (segment (start 141.05 95.875) (end 140.05 95.875) (width 0.2) (layer F.Cu) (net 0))
 (segment (start 141.246 95.679) (end 141.05 95.875) (width 0.2) (layer F.Cu) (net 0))
 (segment (start 135.946 92.624) (end 134.524 92.624) (width 0.2) (layer F.Cu) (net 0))
 (segment (start 134.524 92.624) (end 134.325 92.425) (width 0.2) (layer F.Cu) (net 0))
 (segment (start 135.946 92.224) (end 134.526 92.224) (width 0.2) (layer F.Cu) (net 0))
 (segment (start 134.325 92.425) (end 135.8 92.425) (width 0.2) (layer B.Cu) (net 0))
 (via (at 134.325 92.425) (size 0.6) (drill 0.4) (layers F.Cu B.Cu) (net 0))
 (segment (start 134.526 92.224) (end 134.325 92.425) (width 0.2) (layer F.Cu) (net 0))
 (segment (start 135.946 90.624) (end 134.524 90.624) (width 0.2) (layer F.Cu) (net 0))
 (segment (start 134.524 90.624) (end 134.325 90.425) (width 0.2) (layer F.Cu) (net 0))
 (segment (start 135.946 90.224) (end 134.526 90.224) (width 0.2) (layer F.Cu) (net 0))
 (segment (start 134.526 90.224) (end 134.325 90.425) (width 0.2) (layer F.Cu) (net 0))
 (segment (start 134.325 90.425) (end 135.8 90.425) (width 0.2) (layer B.Cu) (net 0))
 (via (at 134.325 90.425) (size 0.6) (drill 0.4) (layers F.Cu B.Cu) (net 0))
 (segment (start 137.3 92.425) (end 137.445 92.425) (width 0.25) (layer B.Cu) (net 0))
 (segment (start 137.445 92.425) (end 139.446 90.424) (width 0.25) (layer B.Cu) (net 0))
 (segment (start 137.3 90.425) (end 139.445 90.425) (width 0.25) (layer B.Cu) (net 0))
 (segment (start 139.445 90.425) (end 139.446 90.424) (width 0.25) (layer B.Cu) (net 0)))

